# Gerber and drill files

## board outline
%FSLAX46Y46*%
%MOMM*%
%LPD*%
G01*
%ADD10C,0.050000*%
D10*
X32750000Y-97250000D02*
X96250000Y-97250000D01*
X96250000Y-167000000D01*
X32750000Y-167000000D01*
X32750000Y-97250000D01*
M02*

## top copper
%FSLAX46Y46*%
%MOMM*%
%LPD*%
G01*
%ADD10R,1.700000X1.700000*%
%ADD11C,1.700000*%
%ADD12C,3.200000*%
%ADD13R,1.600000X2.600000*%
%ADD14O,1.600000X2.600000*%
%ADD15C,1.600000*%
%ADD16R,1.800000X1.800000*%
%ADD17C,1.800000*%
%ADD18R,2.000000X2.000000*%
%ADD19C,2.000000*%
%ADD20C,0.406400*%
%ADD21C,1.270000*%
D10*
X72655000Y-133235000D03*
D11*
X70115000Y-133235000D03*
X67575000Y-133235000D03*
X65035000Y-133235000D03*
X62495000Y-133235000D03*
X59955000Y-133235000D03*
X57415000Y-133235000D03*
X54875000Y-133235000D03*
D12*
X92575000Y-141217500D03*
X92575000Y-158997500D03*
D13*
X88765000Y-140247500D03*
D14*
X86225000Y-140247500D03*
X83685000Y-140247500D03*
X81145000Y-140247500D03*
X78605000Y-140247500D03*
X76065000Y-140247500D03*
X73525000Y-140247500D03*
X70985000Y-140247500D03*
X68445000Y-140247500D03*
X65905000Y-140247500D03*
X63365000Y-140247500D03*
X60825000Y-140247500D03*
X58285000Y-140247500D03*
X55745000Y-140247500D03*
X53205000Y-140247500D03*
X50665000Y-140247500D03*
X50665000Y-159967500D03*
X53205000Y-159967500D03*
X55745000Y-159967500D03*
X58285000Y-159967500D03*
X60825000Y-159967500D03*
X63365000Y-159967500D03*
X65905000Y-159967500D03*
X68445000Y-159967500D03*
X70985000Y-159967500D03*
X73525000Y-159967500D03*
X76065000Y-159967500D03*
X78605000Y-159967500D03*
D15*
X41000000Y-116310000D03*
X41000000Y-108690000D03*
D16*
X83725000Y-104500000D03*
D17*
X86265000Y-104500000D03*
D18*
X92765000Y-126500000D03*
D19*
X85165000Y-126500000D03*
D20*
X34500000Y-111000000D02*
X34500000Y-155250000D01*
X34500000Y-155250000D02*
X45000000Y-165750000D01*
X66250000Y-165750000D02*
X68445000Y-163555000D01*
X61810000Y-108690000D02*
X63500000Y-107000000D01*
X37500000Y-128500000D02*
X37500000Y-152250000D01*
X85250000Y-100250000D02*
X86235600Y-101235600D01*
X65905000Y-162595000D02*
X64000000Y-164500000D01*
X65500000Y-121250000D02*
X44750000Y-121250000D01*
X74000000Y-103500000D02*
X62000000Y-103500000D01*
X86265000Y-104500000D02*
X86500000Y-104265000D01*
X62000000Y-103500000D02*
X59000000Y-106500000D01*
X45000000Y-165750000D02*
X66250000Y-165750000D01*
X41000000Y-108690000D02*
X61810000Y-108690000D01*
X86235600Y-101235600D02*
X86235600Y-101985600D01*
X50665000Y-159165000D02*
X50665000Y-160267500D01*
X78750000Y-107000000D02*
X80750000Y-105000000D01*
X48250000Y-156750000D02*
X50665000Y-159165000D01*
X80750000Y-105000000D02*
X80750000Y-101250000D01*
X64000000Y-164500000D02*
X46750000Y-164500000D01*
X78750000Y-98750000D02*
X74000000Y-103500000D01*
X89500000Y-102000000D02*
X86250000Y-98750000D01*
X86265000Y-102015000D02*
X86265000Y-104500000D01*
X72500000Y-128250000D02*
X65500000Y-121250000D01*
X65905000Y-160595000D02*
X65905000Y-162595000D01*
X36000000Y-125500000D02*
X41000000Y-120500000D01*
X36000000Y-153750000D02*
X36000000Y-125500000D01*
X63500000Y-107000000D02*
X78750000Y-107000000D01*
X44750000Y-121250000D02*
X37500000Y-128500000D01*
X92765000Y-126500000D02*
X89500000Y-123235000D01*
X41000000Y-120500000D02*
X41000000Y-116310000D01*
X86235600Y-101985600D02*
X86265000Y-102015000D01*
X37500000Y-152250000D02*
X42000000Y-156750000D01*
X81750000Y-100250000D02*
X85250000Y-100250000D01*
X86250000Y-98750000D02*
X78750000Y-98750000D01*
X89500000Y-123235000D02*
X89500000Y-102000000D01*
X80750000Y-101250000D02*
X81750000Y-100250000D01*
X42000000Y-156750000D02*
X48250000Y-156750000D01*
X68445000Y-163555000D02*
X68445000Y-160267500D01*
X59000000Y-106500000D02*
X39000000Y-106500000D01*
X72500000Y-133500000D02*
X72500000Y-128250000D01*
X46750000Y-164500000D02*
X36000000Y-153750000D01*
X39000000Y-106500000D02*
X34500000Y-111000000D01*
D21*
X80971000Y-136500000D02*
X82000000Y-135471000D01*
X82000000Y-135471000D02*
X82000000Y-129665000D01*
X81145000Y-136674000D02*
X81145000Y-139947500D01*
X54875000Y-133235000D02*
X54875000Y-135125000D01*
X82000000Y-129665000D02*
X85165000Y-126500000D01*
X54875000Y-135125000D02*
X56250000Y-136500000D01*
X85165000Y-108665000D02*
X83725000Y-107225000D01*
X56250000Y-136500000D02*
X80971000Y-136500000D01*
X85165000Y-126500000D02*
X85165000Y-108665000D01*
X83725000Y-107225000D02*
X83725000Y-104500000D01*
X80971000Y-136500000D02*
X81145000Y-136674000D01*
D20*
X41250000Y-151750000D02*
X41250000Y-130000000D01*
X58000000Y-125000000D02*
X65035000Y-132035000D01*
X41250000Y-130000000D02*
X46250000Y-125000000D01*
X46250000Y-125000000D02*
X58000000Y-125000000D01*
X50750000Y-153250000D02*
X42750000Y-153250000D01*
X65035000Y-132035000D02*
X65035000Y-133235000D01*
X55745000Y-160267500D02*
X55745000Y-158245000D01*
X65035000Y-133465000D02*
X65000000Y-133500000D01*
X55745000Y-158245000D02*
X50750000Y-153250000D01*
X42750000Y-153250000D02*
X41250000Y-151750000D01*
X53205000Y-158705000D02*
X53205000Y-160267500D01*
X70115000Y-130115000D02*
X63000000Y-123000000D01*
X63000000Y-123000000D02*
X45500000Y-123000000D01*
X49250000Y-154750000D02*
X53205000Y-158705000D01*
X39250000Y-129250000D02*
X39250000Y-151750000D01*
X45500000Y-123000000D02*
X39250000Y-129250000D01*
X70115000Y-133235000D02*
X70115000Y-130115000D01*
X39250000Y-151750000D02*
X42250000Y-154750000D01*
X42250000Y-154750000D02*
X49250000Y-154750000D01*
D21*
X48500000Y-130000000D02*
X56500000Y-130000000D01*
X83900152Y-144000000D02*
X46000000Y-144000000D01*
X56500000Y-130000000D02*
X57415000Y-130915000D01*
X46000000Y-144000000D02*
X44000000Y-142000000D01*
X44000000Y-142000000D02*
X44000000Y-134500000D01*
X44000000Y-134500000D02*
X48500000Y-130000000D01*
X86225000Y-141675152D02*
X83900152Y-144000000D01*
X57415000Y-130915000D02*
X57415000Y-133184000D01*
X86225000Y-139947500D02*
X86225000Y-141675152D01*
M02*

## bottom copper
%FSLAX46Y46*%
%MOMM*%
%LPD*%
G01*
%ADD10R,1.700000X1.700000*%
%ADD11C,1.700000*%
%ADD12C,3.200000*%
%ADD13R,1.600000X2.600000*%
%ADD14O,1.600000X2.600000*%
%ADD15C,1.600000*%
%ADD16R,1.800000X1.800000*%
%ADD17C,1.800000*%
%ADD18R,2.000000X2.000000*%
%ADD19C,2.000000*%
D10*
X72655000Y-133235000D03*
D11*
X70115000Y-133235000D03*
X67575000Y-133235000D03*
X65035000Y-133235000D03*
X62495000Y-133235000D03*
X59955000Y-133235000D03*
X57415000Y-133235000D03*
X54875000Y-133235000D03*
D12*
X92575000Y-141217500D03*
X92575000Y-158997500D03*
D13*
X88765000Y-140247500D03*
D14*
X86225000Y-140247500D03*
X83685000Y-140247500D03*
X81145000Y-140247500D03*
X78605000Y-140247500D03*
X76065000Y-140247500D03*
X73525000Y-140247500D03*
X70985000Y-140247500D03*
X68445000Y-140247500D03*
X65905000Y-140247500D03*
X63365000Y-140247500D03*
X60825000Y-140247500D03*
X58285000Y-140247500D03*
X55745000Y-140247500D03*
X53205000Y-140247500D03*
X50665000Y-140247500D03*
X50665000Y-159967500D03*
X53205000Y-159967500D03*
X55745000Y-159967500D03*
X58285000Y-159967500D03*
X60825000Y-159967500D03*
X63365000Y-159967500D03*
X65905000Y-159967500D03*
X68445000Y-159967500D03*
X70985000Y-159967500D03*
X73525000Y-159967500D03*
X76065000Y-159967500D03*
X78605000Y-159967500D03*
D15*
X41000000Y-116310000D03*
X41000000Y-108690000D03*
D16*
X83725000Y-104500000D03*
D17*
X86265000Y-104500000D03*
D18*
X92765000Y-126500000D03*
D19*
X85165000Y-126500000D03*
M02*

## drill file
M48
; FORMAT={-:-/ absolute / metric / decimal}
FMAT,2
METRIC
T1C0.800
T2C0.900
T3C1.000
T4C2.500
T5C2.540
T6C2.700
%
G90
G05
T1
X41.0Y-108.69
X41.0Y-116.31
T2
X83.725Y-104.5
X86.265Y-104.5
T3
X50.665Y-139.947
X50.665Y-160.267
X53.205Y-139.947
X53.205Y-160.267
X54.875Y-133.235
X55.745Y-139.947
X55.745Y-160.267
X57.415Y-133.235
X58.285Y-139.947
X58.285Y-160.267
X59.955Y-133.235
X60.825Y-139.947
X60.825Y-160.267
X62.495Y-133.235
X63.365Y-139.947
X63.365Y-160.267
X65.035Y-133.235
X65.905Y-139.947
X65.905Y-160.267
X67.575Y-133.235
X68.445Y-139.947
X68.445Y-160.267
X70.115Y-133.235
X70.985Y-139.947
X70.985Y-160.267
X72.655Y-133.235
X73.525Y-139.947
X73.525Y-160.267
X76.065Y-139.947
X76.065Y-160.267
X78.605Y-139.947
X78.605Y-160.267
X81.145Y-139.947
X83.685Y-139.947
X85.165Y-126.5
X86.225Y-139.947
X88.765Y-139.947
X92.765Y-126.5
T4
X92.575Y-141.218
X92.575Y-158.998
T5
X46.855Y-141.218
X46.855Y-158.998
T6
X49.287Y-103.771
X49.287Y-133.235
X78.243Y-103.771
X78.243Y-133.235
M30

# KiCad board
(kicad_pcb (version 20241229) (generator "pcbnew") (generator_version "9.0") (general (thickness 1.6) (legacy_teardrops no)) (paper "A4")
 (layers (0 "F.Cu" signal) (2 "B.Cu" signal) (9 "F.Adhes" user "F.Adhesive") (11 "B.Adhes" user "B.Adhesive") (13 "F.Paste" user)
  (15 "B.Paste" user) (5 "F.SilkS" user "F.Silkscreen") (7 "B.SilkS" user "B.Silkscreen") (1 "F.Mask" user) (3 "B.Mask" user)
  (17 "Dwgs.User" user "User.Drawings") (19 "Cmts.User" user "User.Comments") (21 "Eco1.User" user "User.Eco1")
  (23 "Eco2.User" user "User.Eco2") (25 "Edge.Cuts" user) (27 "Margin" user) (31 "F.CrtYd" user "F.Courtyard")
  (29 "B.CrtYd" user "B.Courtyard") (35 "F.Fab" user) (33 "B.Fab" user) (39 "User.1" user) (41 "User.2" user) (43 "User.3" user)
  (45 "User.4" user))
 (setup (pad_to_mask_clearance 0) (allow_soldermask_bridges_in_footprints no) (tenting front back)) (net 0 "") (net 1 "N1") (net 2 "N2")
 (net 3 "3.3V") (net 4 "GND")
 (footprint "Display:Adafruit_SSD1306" (layer "F.Cu") (at 72.655 133.235 180)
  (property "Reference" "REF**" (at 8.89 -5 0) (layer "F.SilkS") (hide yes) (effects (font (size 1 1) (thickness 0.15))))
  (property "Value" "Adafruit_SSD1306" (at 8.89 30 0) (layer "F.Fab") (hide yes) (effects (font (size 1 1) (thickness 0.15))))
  (pad "" np_thru_hole circle (at -5.588 0 180) (size 2.7 2.7) (drill 2.7) (layers "*.Cu" "*.Mask"))
  (pad "" np_thru_hole circle (at -5.588 29.464 180) (size 2.7 2.7) (drill 2.7) (layers "*.Cu" "*.Mask"))
  (pad "" np_thru_hole circle (at 23.368 0 180) (size 2.7 2.7) (drill 2.7) (layers "*.Cu" "*.Mask"))
  (pad "" np_thru_hole circle (at 23.368 29.464 180) (size 2.7 2.7) (drill 2.7) (layers "*.Cu" "*.Mask"))
  (pad "1" thru_hole rect (at 0 0 180) (size 1.7 1.7) (drill 1) (layers "*.Cu" "*.Mask") (remove_unused_layers no))
  (pad "2" thru_hole circle (at 2.54 0 180) (size 1.7 1.7) (drill 1) (layers "*.Cu" "*.Mask") (remove_unused_layers no) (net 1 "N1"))
  (pad "3" thru_hole circle (at 5.08 0 180) (size 1.7 1.7) (drill 1) (layers "*.Cu" "*.Mask") (remove_unused_layers no))
  (pad "4" thru_hole circle (at 7.62 0 180) (size 1.7 1.7) (drill 1) (layers "*.Cu" "*.Mask") (remove_unused_layers no) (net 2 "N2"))
  (pad "5" thru_hole circle (at 10.16 0 180) (size 1.7 1.7) (drill 1) (layers "*.Cu" "*.Mask") (remove_unused_layers no))
  (pad "6" thru_hole circle (at 12.7 0 180) (size 1.7 1.7) (drill 1) (layers "*.Cu" "*.Mask") (remove_unused_layers no))
  (pad "7" thru_hole circle (at 15.24 0 180) (size 1.7 1.7) (drill 1) (layers "*.Cu" "*.Mask") (remove_unused_layers no) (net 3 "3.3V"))
  (pad "8" thru_hole circle (at 17.78 0 180) (size 1.7 1.7) (drill 1) (layers "*.Cu" "*.Mask") (remove_unused_layers no) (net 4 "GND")))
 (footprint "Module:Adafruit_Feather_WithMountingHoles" (layer "F.Cu") (at 88.765 139.9475 -90)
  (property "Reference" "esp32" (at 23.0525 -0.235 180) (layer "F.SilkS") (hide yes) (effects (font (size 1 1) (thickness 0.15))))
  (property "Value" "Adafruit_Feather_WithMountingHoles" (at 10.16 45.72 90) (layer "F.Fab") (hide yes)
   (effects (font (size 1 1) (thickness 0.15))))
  (pad "" np_thru_hole circle (at 1.27 -3.81 180) (size 3.2 3.2) (drill 2.5) (layers "*.Cu" "*.Mask"))
  (pad "" np_thru_hole circle (at 1.27 41.91 180) (size 2.54 2.54) (drill 2.54) (layers "*.Cu" "*.Mask"))
  (pad "" np_thru_hole circle (at 19.05 -3.81 180) (size 3.2 3.2) (drill 2.5) (layers "*.Cu" "*.Mask"))
  (pad "" np_thru_hole circle (at 19.05 41.91 180) (size 2.54 2.54) (drill 2.54) (layers "*.Cu" "*.Mask"))
  (pad "1" thru_hole rect (at 0 0 270) (size 2.6 1.6) (drill 1 (offset 0.3 0)) (layers "*.Cu" "*.Mask") (remove_unused_layers no))
  (pad "2" thru_hole oval (at 0 2.54 270) (size 2.6 1.6) (drill 1 (offset 0.3 0)) (layers "*.Cu" "*.Mask") (remove_unused_layers no)
   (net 3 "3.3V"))
  (pad "3" thru_hole oval (at 0 5.08 270) (size 2.6 1.6) (drill 1 (offset 0.3 0)) (layers "*.Cu" "*.Mask") (remove_unused_layers no))
  (pad "4" thru_hole oval (at 0 7.62 270) (size 2.6 1.6) (drill 1 (offset 0.3 0)) (layers "*.Cu" "*.Mask") (remove_unused_layers no)
   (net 4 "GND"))
  (pad "5" thru_hole oval (at 0 10.16 270) (size 2.6 1.6) (drill 1 (offset 0.3 0)) (layers "*.Cu" "*.Mask") (remove_unused_layers no))
  (pad "6" thru_hole oval (at 0 12.7 270) (size 2.6 1.6) (drill 1 (offset 0.3 0)) (layers "*.Cu" "*.Mask") (remove_unused_layers no))
  (pad "7" thru_hole oval (at 0 15.24 270) (size 2.6 1.6) (drill 1 (offset 0.3 0)) (layers "*.Cu" "*.Mask") (remove_unused_layers no))
  (pad "8" thru_hole oval (at 0 17.78 270) (size 2.6 1.6) (drill 1 (offset 0.3 0)) (layers "*.Cu" "*.Mask") (remove_unused_layers no))
  (pad "9" thru_hole oval (at 0 20.32 270) (size 2.6 1.6) (drill 1 (offset 0.3 0)) (layers "*.Cu" "*.Mask") (remove_unused_layers no))
  (pad "10" thru_hole oval (at 0 22.86 270) (size 2.6 1.6) (drill 1 (offset 0.3 0)) (layers "*.Cu" "*.Mask") (remove_unused_layers no))
  (pad "11" thru_hole oval (at 0 25.4 270) (size 2.6 1.6) (drill 1 (offset 0.3 0)) (layers "*.Cu" "*.Mask") (remove_unused_layers no))
  (pad "12" thru_hole oval (at 0 27.94 270) (size 2.6 1.6) (drill 1 (offset 0.3 0)) (layers "*.Cu" "*.Mask") (remove_unused_layers no))
  (pad "13" thru_hole oval (at 0 30.48 270) (size 2.6 1.6) (drill 1 (offset 0.3 0)) (layers "*.Cu" "*.Mask") (remove_unused_layers no))
  (pad "14" thru_hole oval (at 0 33.02 270) (size 2.6 1.6) (drill 1 (offset 0.3 0)) (layers "*.Cu" "*.Mask") (remove_unused_layers no))
  (pad "15" thru_hole oval (at 0 35.56 270) (size 2.6 1.6) (drill 1 (offset 0.3 0)) (layers "*.Cu" "*.Mask") (remove_unused_layers no))
  (pad "16" thru_hole oval (at 0 38.1 270) (size 2.6 1.6) (drill 1 (offset 0.3 0)) (layers "*.Cu" "*.Mask") (remove_unused_layers no))
  (pad "17" thru_hole oval (at 20.32 38.1 90) (size 2.6 1.6) (drill 1 (offset 0.3 0)) (layers "*.Cu" "*.Mask") (remove_unused_layers no))
  (pad "18" thru_hole oval (at 20.32 35.56 90) (size 2.6 1.6) (drill 1 (offset 0.3 0)) (layers "*.Cu" "*.Mask") (remove_unused_layers no)
   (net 1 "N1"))
  (pad "19" thru_hole oval (at 20.32 33.02 90) (size 2.6 1.6) (drill 1 (offset 0.3 0)) (layers "*.Cu" "*.Mask") (remove_unused_layers no)
   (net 2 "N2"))
  (pad "20" thru_hole oval (at 20.32 30.48 90) (size 2.6 1.6) (drill 1 (offset 0.3 0)) (layers "*.Cu" "*.Mask") (remove_unused_layers no))
  (pad "21" thru_hole oval (at 20.32 27.94 90) (size 2.6 1.6) (drill 1 (offset 0.3 0)) (layers "*.Cu" "*.Mask") (remove_unused_layers no))
  (pad "22" thru_hole oval (at 20.32 25.4 90) (size 2.6 1.6) (drill 1 (offset 0.3 0)) (layers "*.Cu" "*.Mask") (remove_unused_layers no))
  (pad "23" thru_hole oval (at 20.32 22.86 90) (size 2.6 1.6) (drill 1 (offset 0.3 0)) (layers "*.Cu" "*.Mask") (remove_unused_layers no))
  (pad "24" thru_hole oval (at 20.32 20.32 90) (size 2.6 1.6) (drill 1 (offset 0.3 0)) (layers "*.Cu" "*.Mask") (remove_unused_layers no))
  (pad "25" thru_hole oval (at 20.32 17.78 90) (size 2.6 1.6) (drill 1 (offset 0.3 0)) (layers "*.Cu" "*.Mask") (remove_unused_layers no))
  (pad "26" thru_hole oval (at 20.32 15.24 90) (size 2.6 1.6) (drill 1 (offset 0.3 0)) (layers "*.Cu" "*.Mask") (remove_unused_layers no))
  (pad "27" thru_hole oval (at 20.32 12.7 90) (size 2.6 1.6) (drill 1 (offset 0.3 0)) (layers "*.Cu" "*.Mask") (remove_unused_layers no))
  (pad "28" thru_hole oval (at 20.32 10.16 90) (size 2.6 1.6) (drill 1 (offset 0.3 0)) (layers "*.Cu" "*.Mask") (remove_unused_layers no)))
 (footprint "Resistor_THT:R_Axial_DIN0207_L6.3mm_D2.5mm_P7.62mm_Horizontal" (layer "F.Cu") (at 41 116.31 90)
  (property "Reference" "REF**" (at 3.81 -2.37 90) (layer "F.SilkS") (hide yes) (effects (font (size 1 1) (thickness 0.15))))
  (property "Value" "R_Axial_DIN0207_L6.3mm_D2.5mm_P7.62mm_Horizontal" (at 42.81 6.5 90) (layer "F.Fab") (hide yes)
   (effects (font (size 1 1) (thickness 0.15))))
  (pad "1" thru_hole circle (at 0 0 90) (size 1.6 1.6) (drill 0.8) (layers "*.Cu" "*.Mask") (remove_unused_layers no))
  (pad "2" thru_hole circle (at 7.62 0 90) (size 1.6 1.6) (drill 0.8) (layers "*.Cu" "*.Mask") (remove_unused_layers no)))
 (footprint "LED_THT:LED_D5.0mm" (layer "F.Cu") (at 83.725 104.5)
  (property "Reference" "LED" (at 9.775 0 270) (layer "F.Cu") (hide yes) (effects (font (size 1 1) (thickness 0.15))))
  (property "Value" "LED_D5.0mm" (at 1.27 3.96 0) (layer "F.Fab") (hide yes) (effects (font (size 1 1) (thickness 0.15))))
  (pad "1" thru_hole rect (at 0 0) (size 1.8 1.8) (drill 0.9) (layers "*.Cu" "*.Mask") (remove_unused_layers no) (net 4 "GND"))
  (pad "2" thru_hole circle (at 2.54 0) (size 1.8 1.8) (drill 0.9) (layers "*.Cu" "*.Mask") (remove_unused_layers no)))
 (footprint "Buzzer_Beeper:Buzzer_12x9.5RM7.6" (layer "F.Cu") (at 92.765 126.5 180)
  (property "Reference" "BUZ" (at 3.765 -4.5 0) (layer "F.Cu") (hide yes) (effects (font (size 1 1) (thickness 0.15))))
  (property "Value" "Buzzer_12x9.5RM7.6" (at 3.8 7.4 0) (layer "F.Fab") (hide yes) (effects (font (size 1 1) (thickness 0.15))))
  (pad "1" thru_hole rect (at 0 0 180) (size 2 2) (drill 1) (layers "*.Cu" "*.Mask") (remove_unused_layers no))
  (pad "2" thru_hole circle (at 7.6 0 180) (size 2 2) (drill 1) (layers "*.Cu" "*.Mask") (remove_unused_layers no) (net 4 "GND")))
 (gr_rect (start 32.75 97.25) (end 96.25 167) (stroke (width 0.05) (type default)) (fill no) (layer "Edge.Cuts"))
 (segment (start 34.5 111) (end 34.5 155.25) (width 0.4064) (layer "F.Cu") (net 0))
 (segment (start 34.5 155.25) (end 45 165.75) (width 0.4064) (layer "F.Cu") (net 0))
 (segment (start 66.25 165.75) (end 68.445 163.555) (width 0.4064) (layer "F.Cu") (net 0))
 (segment (start 61.81 108.69) (end 63.5 107) (width 0.4064) (layer "F.Cu") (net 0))
 (segment (start 37.5 128.5) (end 37.5 152.25) (width 0.4064) (layer "F.Cu") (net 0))
 (segment (start 85.25 100.25) (end 86.2356 101.2356) (width 0.4064) (layer "F.Cu") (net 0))
 (segment (start 65.905 162.595) (end 64 164.5) (width 0.4064) (layer "F.Cu") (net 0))
 (segment (start 65.5 121.25) (end 44.75 121.25) (width 0.4064) (layer "F.Cu") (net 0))
 (segment (start 74 103.5) (end 62 103.5) (width 0.4064) (layer "F.Cu") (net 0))
 (segment (start 86.265 104.5) (end 86.5 104.265) (width 0.4064) (layer "F.Cu") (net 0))
 (segment (start 62 103.5) (end 59 106.5) (width 0.4064) (layer "F.Cu") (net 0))
 (segment (start 45 165.75) (end 66.25 165.75) (width 0.4064) (layer "F.Cu") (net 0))
 (segment (start 41 108.69) (end 61.81 108.69) (width 0.4064) (layer "F.Cu") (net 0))
 (segment (start 86.2356 101.2356) (end 86.2356 101.9856) (width 0.4064) (layer "F.Cu") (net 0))
 (segment (start 50.665 159.165) (end 50.665 160.2675) (width 0.4064) (layer "F.Cu") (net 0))
 (segment (start 78.75 107) (end 80.75 105) (width 0.4064) (layer "F.Cu") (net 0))
 (segment (start 48.25 156.75) (end 50.665 159.165) (width 0.4064) (layer "F.Cu") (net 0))
 (segment (start 80.75 105) (end 80.75 101.25) (width 0.4064) (layer "F.Cu") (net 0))
 (segment (start 64 164.5) (end 46.75 164.5) (width 0.4064) (layer "F.Cu") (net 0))
 (segment (start 78.75 98.75) (end 74 103.5) (width 0.4064) (layer "F.Cu") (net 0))
 (segment (start 89.5 102) (end 86.25 98.75) (width 0.4064) (layer "F.Cu") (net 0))
 (segment (start 86.265 102.015) (end 86.265 104.5) (width 0.4064) (layer "F.Cu") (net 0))
 (segment (start 72.5 128.25) (end 65.5 121.25) (width 0.4064) (layer "F.Cu") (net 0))
 (segment (start 65.905 160.595) (end 65.905 162.595) (width 0.4064) (layer "F.Cu") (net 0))
 (segment (start 36 125.5) (end 41 120.5) (width 0.4064) (layer "F.Cu") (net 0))
 (segment (start 36 153.75) (end 36 125.5) (width 0.4064) (layer "F.Cu") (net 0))
 (segment (start 63.5 107) (end 78.75 107) (width 0.4064) (layer "F.Cu") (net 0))
 (segment (start 44.75 121.25) (end 37.5 128.5) (width 0.4064) (layer "F.Cu") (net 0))
 (segment (start 92.765 126.5) (end 89.5 123.235) (width 0.4064) (layer "F.Cu") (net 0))
 (segment (start 41 120.5) (end 41 116.31) (width 0.4064) (layer "F.Cu") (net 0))
 (segment (start 86.2356 101.9856) (end 86.265 102.015) (width 0.4064) (layer "F.Cu") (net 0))
 (segment (start 37.5 152.25) (end 42 156.75) (width 0.4064) (layer "F.Cu") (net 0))
 (segment (start 81.75 100.25) (end 85.25 100.25) (width 0.4064) (layer "F.Cu") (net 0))
 (segment (start 86.25 98.75) (end 78.75 98.75) (width 0.4064) (layer "F.Cu") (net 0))
 (segment (start 89.5 123.235) (end 89.5 102) (width 0.4064) (layer "F.Cu") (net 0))
 (segment (start 80.75 101.25) (end 81.75 100.25) (width 0.4064) (layer "F.Cu") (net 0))
 (segment (start 42 156.75) (end 48.25 156.75) (width 0.4064) (layer "F.Cu") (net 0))
 (segment (start 68.445 163.555) (end 68.445 160.2675) (width 0.4064) (layer "F.Cu") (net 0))
 (segment (start 59 106.5) (end 39 106.5) (width 0.4064) (layer "F.Cu") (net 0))
 (segment (start 72.5 133.5) (end 72.5 128.25) (width 0.4064) (layer "F.Cu") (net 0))
 (segment (start 46.75 164.5) (end 36 153.75) (width 0.4064) (layer "F.Cu") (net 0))
 (segment (start 39 106.5) (end 34.5 111) (width 0.4064) (layer "F.Cu") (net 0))
 (segment (start 80.971 136.5) (end 82 135.471) (width 1.27) (layer "F.Cu") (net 4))
 (segment (start 82 135.471) (end 82 129.665) (width 1.27) (layer "F.Cu") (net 4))
 (segment (start 81.145 136.674) (end 81.145 139.9475) (width 1.27) (layer "F.Cu") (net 4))
 (segment (start 54.875 133.235) (end 54.875 135.125) (width 1.27) (layer "F.Cu") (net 4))
 (segment (start 82 129.665) (end 85.165 126.5) (width 1.27) (layer "F.Cu") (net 4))
 (segment (start 54.875 135.125) (end 56.25 136.5) (width 1.27) (layer "F.Cu") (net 4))
 (segment (start 85.165 108.665) (end 83.725 107.225) (width 1.27) (layer "F.Cu") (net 4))
 (segment (start 56.25 136.5) (end 80.971 136.5) (width 1.27) (layer "F.Cu") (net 4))
 (segment (start 85.165 126.5) (end 85.165 108.665) (width 1.27) (layer "F.Cu") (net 4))
 (segment (start 83.725 107.225) (end 83.725 104.5) (width 1.27) (layer "F.Cu") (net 4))
 (segment (start 80.971 136.5) (end 81.145 136.674) (width 1.27) (layer "F.Cu") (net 4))
 (segment (start 41.25 151.75) (end 41.25 130) (width 0.4064) (layer "F.Cu") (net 2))
 (segment (start 58 125) (end 65.035 132.035) (width 0.4064) (layer "F.Cu") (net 2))
 (segment (start 41.25 130) (end 46.25 125) (width 0.4064) (layer "F.Cu") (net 2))
 (segment (start 46.25 125) (end 58 125) (width 0.4064) (layer "F.Cu") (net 2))
 (segment (start 50.75 153.25) (end 42.75 153.25) (width 0.4064) (layer "F.Cu") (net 2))
 (segment (start 65.035 132.035) (end 65.035 133.235) (width 0.4064) (layer "F.Cu") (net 2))
 (segment (start 55.745 160.2675) (end 55.745 158.245) (width 0.4064) (layer "F.Cu") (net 2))
 (segment (start 65.035 133.465) (end 65 133.5) (width 0.4064) (layer "F.Cu") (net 2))
 (segment (start 55.745 158.245) (end 50.75 153.25) (width 0.4064) (layer "F.Cu") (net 2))
 (segment (start 42.75 153.25) (end 41.25 151.75) (width 0.4064) (layer "F.Cu") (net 2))
 (segment (start 53.205 158.705) (end 53.205 160.2675) (width 0.4064) (layer "F.Cu") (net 1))
 (segment (start 70.115 130.115) (end 63 123) (width 0.4064) (layer "F.Cu") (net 1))
 (segment (start 63 123) (end 45.5 123) (width 0.4064) (layer "F.Cu") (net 1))
 (segment (start 49.25 154.75) (end 53.205 158.705) (width 0.4064) (layer "F.Cu") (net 1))
 (segment (start 39.25 129.25) (end 39.25 151.75) (width 0.4064) (layer "F.Cu") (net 1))
 (segment (start 45.5 123) (end 39.25 129.25) (width 0.4064) (layer "F.Cu") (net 1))
 (segment (start 70.115 133.235) (end 70.115 130.115) (width 0.4064) (layer "F.Cu") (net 1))
 (segment (start 39.25 151.75) (end 42.25 154.75) (width 0.4064) (layer "F.Cu") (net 1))
 (segment (start 42.25 154.75) (end 49.25 154.75) (width 0.4064) (layer "F.Cu") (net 1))
 (segment (start 48.5 130) (end 56.5 130) (width 1.27) (layer "F.Cu") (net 3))
 (segment (start 83.900152 144) (end 46 144) (width 1.27) (layer "F.Cu") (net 3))
 (segment (start 56.5 130) (end 57.415 130.915) (width 1.27) (layer "F.Cu") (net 3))
 (segment (start 46 144) (end 44 142) (width 1.27) (layer "F.Cu") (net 3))
 (segment (start 44 142) (end 44 134.5) (width 1.27) (layer "F.Cu") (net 3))
 (segment (start 44 134.5) (end 48.5 130) (width 1.27) (layer "F.Cu") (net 3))
 (segment (start 86.225 141.675152) (end 83.900152 144) (width 1.27) (layer "F.Cu") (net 3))
 (segment (start 57.415 130.915) (end 57.415 133.184) (width 1.27) (layer "F.Cu") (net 3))
 (segment (start 86.225 139.9475) (end 86.225 141.675152) (width 1.27) (layer "F.Cu") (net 3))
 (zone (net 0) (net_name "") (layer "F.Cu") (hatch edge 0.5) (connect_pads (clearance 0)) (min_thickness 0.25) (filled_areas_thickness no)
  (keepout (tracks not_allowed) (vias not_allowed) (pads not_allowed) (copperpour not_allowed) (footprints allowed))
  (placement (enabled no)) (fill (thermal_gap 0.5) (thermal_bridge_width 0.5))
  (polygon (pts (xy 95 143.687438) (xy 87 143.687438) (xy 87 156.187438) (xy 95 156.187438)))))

